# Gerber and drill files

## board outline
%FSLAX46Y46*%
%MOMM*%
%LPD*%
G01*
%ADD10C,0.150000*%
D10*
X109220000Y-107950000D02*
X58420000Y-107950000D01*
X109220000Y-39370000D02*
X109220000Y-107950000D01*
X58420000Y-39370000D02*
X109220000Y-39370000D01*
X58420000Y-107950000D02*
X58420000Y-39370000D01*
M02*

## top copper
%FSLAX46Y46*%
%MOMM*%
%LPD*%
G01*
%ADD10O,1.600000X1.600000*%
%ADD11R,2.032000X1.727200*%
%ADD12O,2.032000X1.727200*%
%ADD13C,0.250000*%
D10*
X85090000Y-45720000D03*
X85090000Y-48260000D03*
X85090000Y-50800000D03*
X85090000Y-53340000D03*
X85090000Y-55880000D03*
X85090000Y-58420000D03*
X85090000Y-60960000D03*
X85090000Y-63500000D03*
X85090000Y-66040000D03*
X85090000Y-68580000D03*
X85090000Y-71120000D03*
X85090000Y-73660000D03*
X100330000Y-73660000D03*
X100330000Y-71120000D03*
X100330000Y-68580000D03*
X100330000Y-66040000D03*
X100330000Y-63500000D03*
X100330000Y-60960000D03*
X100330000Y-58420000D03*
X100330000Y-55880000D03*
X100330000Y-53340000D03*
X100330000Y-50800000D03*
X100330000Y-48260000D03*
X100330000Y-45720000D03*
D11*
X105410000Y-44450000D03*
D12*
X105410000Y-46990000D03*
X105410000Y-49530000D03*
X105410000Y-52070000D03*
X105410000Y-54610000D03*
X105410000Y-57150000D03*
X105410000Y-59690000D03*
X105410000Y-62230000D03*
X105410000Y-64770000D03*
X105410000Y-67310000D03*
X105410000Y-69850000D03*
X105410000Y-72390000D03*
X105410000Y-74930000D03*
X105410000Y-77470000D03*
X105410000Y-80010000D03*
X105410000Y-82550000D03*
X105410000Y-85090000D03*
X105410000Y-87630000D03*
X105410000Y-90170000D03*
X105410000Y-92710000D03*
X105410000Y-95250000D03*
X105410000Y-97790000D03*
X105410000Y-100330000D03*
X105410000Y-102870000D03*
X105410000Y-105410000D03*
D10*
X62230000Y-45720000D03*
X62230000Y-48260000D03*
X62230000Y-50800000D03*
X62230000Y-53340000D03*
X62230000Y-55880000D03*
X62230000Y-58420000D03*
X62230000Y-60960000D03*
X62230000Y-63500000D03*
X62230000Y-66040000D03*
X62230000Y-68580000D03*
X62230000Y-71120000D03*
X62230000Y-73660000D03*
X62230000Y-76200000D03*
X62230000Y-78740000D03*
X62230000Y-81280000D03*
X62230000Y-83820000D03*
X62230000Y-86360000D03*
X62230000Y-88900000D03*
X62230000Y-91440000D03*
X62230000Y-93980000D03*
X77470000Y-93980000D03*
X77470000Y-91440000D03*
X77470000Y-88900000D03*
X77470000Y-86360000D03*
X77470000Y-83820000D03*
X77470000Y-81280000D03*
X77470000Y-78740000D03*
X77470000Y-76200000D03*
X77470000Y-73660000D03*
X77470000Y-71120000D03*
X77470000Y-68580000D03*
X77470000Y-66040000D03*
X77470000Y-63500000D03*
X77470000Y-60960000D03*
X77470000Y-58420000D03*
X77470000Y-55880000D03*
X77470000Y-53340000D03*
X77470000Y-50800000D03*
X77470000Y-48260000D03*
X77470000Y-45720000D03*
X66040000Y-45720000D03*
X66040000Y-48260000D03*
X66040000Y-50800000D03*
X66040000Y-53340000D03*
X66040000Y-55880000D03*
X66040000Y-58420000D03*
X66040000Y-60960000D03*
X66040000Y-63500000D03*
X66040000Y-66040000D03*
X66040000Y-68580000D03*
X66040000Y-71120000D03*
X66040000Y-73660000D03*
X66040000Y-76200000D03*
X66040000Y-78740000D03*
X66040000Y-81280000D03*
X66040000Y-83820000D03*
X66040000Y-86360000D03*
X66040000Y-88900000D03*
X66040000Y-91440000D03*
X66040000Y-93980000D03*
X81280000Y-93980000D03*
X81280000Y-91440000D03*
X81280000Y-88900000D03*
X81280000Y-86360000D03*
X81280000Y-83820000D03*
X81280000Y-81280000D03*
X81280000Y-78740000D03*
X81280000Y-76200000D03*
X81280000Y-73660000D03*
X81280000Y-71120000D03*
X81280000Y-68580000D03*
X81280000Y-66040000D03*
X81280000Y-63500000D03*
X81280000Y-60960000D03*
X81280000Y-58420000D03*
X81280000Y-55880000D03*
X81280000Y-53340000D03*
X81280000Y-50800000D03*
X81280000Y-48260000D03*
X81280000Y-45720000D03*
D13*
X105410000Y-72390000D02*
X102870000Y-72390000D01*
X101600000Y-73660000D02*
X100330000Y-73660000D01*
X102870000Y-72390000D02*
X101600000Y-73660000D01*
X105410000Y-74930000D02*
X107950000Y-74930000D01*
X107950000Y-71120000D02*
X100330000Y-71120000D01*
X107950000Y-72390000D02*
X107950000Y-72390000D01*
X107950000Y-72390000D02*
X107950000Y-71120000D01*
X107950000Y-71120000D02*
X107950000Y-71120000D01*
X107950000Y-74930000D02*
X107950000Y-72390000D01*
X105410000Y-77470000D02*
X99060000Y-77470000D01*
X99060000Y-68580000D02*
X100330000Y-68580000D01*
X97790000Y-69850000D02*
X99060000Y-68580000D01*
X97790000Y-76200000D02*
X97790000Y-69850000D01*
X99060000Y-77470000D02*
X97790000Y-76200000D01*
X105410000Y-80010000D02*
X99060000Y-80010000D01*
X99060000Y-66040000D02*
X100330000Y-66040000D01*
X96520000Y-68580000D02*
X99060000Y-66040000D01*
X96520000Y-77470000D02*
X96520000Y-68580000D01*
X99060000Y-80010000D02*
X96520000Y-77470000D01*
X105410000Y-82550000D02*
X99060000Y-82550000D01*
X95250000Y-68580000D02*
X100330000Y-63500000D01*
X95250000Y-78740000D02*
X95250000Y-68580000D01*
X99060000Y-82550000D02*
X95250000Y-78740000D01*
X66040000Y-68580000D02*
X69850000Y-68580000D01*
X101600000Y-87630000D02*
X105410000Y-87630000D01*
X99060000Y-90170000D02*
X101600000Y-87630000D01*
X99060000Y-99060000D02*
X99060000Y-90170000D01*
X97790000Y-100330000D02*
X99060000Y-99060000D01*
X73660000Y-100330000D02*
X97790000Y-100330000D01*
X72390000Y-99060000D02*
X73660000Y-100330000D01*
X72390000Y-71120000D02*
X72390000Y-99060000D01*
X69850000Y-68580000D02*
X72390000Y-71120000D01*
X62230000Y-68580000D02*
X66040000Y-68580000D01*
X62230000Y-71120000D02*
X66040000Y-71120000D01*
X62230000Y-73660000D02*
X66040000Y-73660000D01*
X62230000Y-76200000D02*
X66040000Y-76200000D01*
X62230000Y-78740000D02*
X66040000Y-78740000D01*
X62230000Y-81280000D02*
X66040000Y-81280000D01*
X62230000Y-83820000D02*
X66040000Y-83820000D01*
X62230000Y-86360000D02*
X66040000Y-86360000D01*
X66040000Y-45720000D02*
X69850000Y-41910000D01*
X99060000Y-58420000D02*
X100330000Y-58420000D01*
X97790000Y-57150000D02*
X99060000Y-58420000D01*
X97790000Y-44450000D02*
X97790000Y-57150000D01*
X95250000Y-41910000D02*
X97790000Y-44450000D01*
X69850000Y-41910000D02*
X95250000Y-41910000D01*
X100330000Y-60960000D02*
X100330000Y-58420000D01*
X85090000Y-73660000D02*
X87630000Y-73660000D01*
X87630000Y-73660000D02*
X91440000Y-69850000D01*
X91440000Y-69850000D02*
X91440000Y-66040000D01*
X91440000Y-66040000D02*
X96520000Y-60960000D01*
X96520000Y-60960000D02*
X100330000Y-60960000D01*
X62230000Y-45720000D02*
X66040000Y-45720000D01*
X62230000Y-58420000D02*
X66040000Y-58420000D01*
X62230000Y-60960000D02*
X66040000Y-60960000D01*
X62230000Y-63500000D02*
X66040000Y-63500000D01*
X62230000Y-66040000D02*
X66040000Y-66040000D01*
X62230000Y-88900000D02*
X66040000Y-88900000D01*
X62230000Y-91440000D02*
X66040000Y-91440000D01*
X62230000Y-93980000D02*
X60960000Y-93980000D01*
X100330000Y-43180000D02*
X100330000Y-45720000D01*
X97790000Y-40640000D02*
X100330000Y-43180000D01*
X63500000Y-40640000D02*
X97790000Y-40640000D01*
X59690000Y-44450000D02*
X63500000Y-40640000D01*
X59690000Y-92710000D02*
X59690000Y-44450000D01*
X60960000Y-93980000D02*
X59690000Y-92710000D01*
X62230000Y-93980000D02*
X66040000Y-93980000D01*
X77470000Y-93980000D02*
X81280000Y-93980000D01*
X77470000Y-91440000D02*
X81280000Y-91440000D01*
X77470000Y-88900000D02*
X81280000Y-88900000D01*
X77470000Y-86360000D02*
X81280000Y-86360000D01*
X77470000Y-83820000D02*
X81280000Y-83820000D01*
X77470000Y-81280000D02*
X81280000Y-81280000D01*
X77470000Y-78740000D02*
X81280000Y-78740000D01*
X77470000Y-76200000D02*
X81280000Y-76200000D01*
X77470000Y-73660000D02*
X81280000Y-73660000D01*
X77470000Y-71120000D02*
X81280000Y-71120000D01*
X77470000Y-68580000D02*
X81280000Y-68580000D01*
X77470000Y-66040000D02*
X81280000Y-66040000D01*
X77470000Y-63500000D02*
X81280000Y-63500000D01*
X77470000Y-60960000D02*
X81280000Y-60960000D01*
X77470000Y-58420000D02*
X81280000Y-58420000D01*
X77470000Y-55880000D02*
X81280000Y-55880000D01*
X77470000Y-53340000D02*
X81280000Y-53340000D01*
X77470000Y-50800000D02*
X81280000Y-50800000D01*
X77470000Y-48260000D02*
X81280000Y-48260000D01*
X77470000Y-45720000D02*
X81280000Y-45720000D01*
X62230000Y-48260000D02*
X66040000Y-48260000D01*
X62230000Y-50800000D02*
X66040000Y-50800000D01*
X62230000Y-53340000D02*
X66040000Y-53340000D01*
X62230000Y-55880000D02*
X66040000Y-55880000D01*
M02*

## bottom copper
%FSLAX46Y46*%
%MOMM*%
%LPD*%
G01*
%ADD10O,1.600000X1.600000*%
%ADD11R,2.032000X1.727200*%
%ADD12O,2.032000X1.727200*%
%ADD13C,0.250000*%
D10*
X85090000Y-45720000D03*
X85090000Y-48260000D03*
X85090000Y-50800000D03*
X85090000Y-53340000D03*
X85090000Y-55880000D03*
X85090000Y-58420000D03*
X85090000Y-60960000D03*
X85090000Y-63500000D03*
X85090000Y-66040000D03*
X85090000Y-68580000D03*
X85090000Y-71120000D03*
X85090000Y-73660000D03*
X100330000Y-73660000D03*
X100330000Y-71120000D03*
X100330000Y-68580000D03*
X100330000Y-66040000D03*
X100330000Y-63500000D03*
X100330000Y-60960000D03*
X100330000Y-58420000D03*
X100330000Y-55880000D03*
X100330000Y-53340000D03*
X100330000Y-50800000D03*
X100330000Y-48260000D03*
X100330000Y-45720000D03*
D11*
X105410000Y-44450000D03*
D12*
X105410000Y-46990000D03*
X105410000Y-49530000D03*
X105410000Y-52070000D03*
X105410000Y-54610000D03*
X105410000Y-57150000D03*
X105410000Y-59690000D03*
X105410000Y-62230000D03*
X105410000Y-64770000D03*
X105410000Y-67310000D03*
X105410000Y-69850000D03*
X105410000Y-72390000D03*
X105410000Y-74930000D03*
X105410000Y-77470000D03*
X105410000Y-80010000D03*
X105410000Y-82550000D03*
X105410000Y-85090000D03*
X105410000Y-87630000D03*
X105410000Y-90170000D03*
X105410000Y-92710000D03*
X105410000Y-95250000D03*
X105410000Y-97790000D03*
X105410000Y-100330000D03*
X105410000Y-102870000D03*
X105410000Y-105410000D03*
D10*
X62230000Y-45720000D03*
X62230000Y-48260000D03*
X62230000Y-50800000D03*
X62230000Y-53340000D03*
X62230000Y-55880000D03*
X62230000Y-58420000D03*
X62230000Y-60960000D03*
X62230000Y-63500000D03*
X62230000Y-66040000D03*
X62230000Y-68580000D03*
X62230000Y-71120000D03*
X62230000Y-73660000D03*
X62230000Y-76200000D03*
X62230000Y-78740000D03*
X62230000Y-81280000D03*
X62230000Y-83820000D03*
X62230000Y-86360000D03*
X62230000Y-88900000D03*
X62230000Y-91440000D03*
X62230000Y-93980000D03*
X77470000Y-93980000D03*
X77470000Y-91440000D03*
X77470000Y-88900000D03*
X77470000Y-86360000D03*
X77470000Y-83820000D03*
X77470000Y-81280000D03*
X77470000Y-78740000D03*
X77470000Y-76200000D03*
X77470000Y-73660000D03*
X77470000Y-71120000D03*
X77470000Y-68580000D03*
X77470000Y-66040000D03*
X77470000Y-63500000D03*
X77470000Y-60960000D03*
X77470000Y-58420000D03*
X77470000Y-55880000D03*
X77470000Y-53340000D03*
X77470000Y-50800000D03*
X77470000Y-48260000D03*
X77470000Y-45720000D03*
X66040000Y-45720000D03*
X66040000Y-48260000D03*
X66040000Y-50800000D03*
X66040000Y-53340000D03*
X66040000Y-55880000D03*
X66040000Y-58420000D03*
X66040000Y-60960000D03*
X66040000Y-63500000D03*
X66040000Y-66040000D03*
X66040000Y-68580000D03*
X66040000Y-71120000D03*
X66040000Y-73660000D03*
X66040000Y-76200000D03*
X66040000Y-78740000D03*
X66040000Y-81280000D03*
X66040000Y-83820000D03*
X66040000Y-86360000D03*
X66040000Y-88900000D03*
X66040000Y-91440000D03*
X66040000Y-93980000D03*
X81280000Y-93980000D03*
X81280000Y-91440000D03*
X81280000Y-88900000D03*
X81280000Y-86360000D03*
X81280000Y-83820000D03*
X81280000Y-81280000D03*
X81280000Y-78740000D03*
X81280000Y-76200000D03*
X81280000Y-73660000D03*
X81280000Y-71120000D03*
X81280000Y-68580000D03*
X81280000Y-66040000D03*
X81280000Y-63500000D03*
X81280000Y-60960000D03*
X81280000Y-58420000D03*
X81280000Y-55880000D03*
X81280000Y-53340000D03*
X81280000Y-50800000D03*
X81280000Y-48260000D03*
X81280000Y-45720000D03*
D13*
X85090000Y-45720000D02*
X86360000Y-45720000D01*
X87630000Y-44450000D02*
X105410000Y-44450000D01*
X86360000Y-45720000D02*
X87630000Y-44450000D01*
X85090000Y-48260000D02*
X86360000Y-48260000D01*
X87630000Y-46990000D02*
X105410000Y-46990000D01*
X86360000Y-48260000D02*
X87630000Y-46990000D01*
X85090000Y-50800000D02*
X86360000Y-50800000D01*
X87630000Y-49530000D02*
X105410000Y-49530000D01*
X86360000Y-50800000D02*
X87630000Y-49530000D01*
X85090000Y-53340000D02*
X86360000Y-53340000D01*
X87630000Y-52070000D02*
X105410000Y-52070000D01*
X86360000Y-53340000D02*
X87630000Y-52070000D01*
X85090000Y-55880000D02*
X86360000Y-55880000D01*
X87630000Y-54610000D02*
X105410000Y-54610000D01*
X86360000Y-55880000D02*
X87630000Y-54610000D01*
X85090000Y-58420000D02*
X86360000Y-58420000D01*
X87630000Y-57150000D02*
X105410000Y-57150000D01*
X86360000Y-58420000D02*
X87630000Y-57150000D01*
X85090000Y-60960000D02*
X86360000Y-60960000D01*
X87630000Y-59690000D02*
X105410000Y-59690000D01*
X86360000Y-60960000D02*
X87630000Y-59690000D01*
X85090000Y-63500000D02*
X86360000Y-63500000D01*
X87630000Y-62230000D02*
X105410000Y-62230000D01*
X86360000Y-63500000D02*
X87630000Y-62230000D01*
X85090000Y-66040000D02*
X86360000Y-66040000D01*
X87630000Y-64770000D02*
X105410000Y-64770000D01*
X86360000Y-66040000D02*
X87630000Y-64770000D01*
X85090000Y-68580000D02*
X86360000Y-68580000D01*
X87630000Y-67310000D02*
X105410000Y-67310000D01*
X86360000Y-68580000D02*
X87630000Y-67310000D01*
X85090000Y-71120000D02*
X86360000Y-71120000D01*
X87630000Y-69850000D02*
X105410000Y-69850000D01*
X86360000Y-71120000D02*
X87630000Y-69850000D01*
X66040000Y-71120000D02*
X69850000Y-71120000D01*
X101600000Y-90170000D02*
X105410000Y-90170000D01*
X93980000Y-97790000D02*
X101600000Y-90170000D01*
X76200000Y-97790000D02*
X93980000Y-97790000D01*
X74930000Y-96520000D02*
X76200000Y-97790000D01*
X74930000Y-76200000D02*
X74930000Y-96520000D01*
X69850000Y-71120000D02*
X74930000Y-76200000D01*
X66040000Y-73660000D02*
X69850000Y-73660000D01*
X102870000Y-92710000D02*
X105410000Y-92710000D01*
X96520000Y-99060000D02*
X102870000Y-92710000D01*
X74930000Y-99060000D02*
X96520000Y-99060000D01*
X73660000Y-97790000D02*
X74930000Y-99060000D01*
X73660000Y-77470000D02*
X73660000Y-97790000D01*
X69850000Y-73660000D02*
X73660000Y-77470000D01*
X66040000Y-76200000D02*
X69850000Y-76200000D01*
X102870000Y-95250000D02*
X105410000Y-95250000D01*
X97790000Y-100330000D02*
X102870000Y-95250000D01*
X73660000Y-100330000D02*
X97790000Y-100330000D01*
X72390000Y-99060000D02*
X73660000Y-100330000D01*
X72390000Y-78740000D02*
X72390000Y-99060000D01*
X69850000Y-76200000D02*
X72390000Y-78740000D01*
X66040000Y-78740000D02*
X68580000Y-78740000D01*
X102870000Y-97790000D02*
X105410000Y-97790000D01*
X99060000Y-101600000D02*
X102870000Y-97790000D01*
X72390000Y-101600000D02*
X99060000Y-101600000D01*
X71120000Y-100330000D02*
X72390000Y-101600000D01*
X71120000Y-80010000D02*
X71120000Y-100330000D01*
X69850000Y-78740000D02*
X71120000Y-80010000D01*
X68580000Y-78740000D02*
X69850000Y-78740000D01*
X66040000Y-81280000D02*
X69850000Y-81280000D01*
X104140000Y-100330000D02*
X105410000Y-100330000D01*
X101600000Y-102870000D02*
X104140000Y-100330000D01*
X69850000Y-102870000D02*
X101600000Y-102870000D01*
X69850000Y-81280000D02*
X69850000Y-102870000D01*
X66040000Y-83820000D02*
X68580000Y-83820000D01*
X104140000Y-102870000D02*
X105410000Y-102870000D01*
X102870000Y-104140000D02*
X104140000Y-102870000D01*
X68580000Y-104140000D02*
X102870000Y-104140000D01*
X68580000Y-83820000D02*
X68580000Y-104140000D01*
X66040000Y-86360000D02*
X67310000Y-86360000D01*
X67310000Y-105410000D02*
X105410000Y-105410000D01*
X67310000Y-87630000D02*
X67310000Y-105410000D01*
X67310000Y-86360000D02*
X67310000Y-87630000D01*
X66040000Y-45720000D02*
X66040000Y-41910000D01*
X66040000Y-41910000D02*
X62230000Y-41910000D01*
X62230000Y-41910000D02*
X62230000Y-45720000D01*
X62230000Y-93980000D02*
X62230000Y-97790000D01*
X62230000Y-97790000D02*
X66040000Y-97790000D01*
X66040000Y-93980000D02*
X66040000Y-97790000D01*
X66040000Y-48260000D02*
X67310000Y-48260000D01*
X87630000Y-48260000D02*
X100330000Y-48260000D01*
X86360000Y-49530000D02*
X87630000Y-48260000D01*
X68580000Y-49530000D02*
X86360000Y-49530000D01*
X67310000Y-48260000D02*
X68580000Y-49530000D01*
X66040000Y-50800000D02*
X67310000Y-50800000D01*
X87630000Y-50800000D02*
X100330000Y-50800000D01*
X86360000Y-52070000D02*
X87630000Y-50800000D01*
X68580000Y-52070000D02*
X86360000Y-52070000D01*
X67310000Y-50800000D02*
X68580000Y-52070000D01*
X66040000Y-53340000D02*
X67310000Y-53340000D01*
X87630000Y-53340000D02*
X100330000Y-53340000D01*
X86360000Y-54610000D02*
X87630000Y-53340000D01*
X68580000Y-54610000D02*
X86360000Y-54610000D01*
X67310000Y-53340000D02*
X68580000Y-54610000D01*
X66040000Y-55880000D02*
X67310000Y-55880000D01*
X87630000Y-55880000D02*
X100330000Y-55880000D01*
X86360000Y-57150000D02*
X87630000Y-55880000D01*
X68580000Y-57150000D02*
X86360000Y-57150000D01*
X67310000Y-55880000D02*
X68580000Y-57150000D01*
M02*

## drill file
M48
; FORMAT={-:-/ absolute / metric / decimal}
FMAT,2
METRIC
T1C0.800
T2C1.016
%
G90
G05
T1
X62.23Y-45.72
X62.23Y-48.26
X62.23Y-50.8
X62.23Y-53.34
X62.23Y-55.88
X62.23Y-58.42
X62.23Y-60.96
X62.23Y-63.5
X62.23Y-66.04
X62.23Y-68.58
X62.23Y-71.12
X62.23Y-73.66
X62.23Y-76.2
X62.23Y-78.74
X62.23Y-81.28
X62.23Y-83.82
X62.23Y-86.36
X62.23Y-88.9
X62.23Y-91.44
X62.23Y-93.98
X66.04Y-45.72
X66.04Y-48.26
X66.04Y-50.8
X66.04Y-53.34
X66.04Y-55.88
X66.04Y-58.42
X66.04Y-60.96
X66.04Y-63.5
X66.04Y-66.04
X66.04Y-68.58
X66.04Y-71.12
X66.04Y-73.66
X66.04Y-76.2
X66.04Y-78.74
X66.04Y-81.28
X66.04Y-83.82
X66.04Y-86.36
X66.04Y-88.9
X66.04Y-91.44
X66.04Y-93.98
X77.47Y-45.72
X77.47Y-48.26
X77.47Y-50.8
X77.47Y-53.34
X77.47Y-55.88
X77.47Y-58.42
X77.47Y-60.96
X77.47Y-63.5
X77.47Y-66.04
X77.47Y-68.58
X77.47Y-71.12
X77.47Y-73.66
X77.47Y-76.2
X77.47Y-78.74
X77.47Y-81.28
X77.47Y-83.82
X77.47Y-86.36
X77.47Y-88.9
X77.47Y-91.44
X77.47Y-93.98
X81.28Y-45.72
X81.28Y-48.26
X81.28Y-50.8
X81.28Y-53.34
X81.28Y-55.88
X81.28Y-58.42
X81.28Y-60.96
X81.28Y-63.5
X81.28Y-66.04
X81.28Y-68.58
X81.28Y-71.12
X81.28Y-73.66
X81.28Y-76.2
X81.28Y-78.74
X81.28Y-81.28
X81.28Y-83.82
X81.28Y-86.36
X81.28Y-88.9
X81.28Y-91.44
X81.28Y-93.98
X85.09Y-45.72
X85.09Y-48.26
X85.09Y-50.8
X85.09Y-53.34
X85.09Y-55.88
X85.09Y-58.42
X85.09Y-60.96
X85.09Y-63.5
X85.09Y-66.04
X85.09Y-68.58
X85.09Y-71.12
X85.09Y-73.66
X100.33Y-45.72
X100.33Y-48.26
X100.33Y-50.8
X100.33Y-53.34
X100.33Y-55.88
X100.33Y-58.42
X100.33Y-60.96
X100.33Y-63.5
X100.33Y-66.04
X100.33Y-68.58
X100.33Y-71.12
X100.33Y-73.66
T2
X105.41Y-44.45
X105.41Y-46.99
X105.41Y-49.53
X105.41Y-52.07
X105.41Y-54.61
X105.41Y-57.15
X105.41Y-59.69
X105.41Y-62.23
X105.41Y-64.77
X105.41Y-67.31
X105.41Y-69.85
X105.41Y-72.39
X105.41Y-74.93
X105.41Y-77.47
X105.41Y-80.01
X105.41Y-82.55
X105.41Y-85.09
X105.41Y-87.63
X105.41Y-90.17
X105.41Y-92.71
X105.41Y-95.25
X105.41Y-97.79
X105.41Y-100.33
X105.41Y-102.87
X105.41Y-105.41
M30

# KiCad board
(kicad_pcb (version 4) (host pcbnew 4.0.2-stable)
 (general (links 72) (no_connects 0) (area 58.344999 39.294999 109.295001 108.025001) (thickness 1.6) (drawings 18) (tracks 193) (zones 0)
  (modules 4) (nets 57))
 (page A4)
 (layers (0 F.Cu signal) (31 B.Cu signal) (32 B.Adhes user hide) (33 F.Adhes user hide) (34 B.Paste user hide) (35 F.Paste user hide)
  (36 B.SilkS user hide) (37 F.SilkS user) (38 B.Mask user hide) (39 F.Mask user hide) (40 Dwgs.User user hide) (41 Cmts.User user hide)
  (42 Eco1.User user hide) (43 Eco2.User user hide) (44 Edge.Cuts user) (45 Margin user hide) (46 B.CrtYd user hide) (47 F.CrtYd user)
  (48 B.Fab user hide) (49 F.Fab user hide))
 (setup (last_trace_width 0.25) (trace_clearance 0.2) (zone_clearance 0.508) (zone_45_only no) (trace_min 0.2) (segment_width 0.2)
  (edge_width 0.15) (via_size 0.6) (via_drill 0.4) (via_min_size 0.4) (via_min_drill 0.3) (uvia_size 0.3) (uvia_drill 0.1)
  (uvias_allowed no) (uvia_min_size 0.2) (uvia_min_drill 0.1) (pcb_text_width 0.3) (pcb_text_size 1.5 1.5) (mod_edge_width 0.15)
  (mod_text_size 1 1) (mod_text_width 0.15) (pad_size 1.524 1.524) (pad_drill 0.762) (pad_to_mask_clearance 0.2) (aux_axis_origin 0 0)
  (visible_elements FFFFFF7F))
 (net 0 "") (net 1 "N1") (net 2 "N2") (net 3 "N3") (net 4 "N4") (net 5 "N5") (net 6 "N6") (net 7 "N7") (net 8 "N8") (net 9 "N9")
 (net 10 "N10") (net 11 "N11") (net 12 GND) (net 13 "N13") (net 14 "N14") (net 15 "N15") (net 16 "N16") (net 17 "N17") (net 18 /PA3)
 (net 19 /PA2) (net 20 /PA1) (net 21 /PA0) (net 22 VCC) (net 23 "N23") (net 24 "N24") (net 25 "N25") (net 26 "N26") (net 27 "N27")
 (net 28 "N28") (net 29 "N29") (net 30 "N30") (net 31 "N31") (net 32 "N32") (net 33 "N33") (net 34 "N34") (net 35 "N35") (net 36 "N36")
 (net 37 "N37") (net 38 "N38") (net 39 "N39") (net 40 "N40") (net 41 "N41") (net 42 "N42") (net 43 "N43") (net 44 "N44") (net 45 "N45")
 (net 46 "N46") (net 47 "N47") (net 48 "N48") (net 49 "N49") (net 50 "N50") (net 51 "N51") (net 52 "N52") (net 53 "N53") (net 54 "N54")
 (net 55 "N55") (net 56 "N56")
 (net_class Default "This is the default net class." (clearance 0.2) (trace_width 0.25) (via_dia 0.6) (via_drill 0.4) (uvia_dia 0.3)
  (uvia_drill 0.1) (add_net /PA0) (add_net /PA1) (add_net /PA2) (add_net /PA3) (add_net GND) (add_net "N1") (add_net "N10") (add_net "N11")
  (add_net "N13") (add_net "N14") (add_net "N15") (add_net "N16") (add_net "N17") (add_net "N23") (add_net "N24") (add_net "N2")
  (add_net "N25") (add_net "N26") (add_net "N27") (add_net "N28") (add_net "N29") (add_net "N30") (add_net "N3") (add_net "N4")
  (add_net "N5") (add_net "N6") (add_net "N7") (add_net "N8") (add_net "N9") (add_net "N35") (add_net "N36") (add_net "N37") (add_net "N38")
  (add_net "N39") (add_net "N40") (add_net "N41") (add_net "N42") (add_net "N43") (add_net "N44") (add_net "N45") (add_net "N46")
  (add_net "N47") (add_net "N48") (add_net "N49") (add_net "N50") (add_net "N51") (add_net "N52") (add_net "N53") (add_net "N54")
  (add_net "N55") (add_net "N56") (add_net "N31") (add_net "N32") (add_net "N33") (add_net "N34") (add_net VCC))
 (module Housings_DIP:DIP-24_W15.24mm (layer F.Cu) (at 85.09 45.72)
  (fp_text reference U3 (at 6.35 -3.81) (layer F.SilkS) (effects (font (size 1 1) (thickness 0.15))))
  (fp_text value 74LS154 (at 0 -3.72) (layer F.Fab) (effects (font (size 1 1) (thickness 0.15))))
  (pad 1 thru_hole oval (at 0 0) (size 1.6 1.6) (drill 0.8) (layers *.Cu *.Mask F.SilkS) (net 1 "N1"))
  (pad 2 thru_hole oval (at 0 2.54) (size 1.6 1.6) (drill 0.8) (layers *.Cu *.Mask F.SilkS) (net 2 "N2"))
  (pad 3 thru_hole oval (at 0 5.08) (size 1.6 1.6) (drill 0.8) (layers *.Cu *.Mask F.SilkS) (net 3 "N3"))
  (pad 4 thru_hole oval (at 0 7.62) (size 1.6 1.6) (drill 0.8) (layers *.Cu *.Mask F.SilkS) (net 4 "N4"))
  (pad 5 thru_hole oval (at 0 10.16) (size 1.6 1.6) (drill 0.8) (layers *.Cu *.Mask F.SilkS) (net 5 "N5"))
  (pad 6 thru_hole oval (at 0 12.7) (size 1.6 1.6) (drill 0.8) (layers *.Cu *.Mask F.SilkS) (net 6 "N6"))
  (pad 7 thru_hole oval (at 0 15.24) (size 1.6 1.6) (drill 0.8) (layers *.Cu *.Mask F.SilkS) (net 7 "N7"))
  (pad 8 thru_hole oval (at 0 17.78) (size 1.6 1.6) (drill 0.8) (layers *.Cu *.Mask F.SilkS) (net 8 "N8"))
  (pad 9 thru_hole oval (at 0 20.32) (size 1.6 1.6) (drill 0.8) (layers *.Cu *.Mask F.SilkS) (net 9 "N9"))
  (pad 10 thru_hole oval (at 0 22.86) (size 1.6 1.6) (drill 0.8) (layers *.Cu *.Mask F.SilkS) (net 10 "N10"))
  (pad 11 thru_hole oval (at 0 25.4) (size 1.6 1.6) (drill 0.8) (layers *.Cu *.Mask F.SilkS) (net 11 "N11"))
  (pad 12 thru_hole oval (at 0 27.94) (size 1.6 1.6) (drill 0.8) (layers *.Cu *.Mask F.SilkS) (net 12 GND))
  (pad 13 thru_hole oval (at 15.24 27.94) (size 1.6 1.6) (drill 0.8) (layers *.Cu *.Mask F.SilkS) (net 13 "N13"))
  (pad 14 thru_hole oval (at 15.24 25.4) (size 1.6 1.6) (drill 0.8) (layers *.Cu *.Mask F.SilkS) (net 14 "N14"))
  (pad 15 thru_hole oval (at 15.24 22.86) (size 1.6 1.6) (drill 0.8) (layers *.Cu *.Mask F.SilkS) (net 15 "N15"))
  (pad 16 thru_hole oval (at 15.24 20.32) (size 1.6 1.6) (drill 0.8) (layers *.Cu *.Mask F.SilkS) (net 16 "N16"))
  (pad 17 thru_hole oval (at 15.24 17.78) (size 1.6 1.6) (drill 0.8) (layers *.Cu *.Mask F.SilkS) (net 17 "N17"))
  (pad 18 thru_hole oval (at 15.24 15.24) (size 1.6 1.6) (drill 0.8) (layers *.Cu *.Mask F.SilkS) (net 12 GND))
  (pad 19 thru_hole oval (at 15.24 12.7) (size 1.6 1.6) (drill 0.8) (layers *.Cu *.Mask F.SilkS) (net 12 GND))
  (pad 20 thru_hole oval (at 15.24 10.16) (size 1.6 1.6) (drill 0.8) (layers *.Cu *.Mask F.SilkS) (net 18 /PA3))
  (pad 21 thru_hole oval (at 15.24 7.62) (size 1.6 1.6) (drill 0.8) (layers *.Cu *.Mask F.SilkS) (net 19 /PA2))
  (pad 22 thru_hole oval (at 15.24 5.08) (size 1.6 1.6) (drill 0.8) (layers *.Cu *.Mask F.SilkS) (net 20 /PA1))
  (pad 23 thru_hole oval (at 15.24 2.54) (size 1.6 1.6) (drill 0.8) (layers *.Cu *.Mask F.SilkS) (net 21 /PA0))
  (pad 24 thru_hole oval (at 15.24 0) (size 1.6 1.6) (drill 0.8) (layers *.Cu *.Mask F.SilkS) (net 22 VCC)))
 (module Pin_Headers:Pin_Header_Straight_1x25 (layer F.Cu) (at 105.41 44.45)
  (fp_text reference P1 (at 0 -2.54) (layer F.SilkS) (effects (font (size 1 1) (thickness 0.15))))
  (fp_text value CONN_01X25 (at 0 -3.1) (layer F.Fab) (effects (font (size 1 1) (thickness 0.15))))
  (pad 1 thru_hole rect (at 0 0) (size 2.032 1.7272) (drill 1.016) (layers *.Cu *.Mask F.SilkS) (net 1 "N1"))
  (pad 2 thru_hole oval (at 0 2.54) (size 2.032 1.7272) (drill 1.016) (layers *.Cu *.Mask F.SilkS) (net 2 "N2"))
  (pad 3 thru_hole oval (at 0 5.08) (size 2.032 1.7272) (drill 1.016) (layers *.Cu *.Mask F.SilkS) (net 3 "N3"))
  (pad 4 thru_hole oval (at 0 7.62) (size 2.032 1.7272) (drill 1.016) (layers *.Cu *.Mask F.SilkS) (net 4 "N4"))
  (pad 5 thru_hole oval (at 0 10.16) (size 2.032 1.7272) (drill 1.016) (layers *.Cu *.Mask F.SilkS) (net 5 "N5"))
  (pad 6 thru_hole oval (at 0 12.7) (size 2.032 1.7272) (drill 1.016) (layers *.Cu *.Mask F.SilkS) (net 6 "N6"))
  (pad 7 thru_hole oval (at 0 15.24) (size 2.032 1.7272) (drill 1.016) (layers *.Cu *.Mask F.SilkS) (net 7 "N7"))
  (pad 8 thru_hole oval (at 0 17.78) (size 2.032 1.7272) (drill 1.016) (layers *.Cu *.Mask F.SilkS) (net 8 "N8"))
  (pad 9 thru_hole oval (at 0 20.32) (size 2.032 1.7272) (drill 1.016) (layers *.Cu *.Mask F.SilkS) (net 9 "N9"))
  (pad 10 thru_hole oval (at 0 22.86) (size 2.032 1.7272) (drill 1.016) (layers *.Cu *.Mask F.SilkS) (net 10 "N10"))
  (pad 11 thru_hole oval (at 0 25.4) (size 2.032 1.7272) (drill 1.016) (layers *.Cu *.Mask F.SilkS) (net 11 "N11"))
  (pad 12 thru_hole oval (at 0 27.94) (size 2.032 1.7272) (drill 1.016) (layers *.Cu *.Mask F.SilkS) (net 13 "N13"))
  (pad 13 thru_hole oval (at 0 30.48) (size 2.032 1.7272) (drill 1.016) (layers *.Cu *.Mask F.SilkS) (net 14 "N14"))
  (pad 14 thru_hole oval (at 0 33.02) (size 2.032 1.7272) (drill 1.016) (layers *.Cu *.Mask F.SilkS) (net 15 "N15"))
  (pad 15 thru_hole oval (at 0 35.56) (size 2.032 1.7272) (drill 1.016) (layers *.Cu *.Mask F.SilkS) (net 16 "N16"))
  (pad 16 thru_hole oval (at 0 38.1) (size 2.032 1.7272) (drill 1.016) (layers *.Cu *.Mask F.SilkS) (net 17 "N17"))
  (pad 17 thru_hole oval (at 0 40.64) (size 2.032 1.7272) (drill 1.016) (layers *.Cu *.Mask F.SilkS))
  (pad 18 thru_hole oval (at 0 43.18) (size 2.032 1.7272) (drill 1.016) (layers *.Cu *.Mask F.SilkS) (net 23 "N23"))
  (pad 19 thru_hole oval (at 0 45.72) (size 2.032 1.7272) (drill 1.016) (layers *.Cu *.Mask F.SilkS) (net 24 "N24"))
  (pad 20 thru_hole oval (at 0 48.26) (size 2.032 1.7272) (drill 1.016) (layers *.Cu *.Mask F.SilkS) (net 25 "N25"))
  (pad 21 thru_hole oval (at 0 50.8) (size 2.032 1.7272) (drill 1.016) (layers *.Cu *.Mask F.SilkS) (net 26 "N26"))
  (pad 22 thru_hole oval (at 0 53.34) (size 2.032 1.7272) (drill 1.016) (layers *.Cu *.Mask F.SilkS) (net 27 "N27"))
  (pad 23 thru_hole oval (at 0 55.88) (size 2.032 1.7272) (drill 1.016) (layers *.Cu *.Mask F.SilkS) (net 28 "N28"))
  (pad 24 thru_hole oval (at 0 58.42) (size 2.032 1.7272) (drill 1.016) (layers *.Cu *.Mask F.SilkS) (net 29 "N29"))
  (pad 25 thru_hole oval (at 0 60.96) (size 2.032 1.7272) (drill 1.016) (layers *.Cu *.Mask F.SilkS) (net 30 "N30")))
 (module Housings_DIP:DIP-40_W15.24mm (layer F.Cu) (at 62.23 45.72)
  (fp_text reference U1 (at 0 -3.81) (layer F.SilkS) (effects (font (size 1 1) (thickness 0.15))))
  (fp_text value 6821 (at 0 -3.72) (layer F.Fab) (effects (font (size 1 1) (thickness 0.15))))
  (pad 1 thru_hole oval (at 0 0) (size 1.6 1.6) (drill 0.8) (layers *.Cu *.Mask F.SilkS) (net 12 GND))
  (pad 2 thru_hole oval (at 0 2.54) (size 1.6 1.6) (drill 0.8) (layers *.Cu *.Mask F.SilkS) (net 21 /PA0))
  (pad 3 thru_hole oval (at 0 5.08) (size 1.6 1.6) (drill 0.8) (layers *.Cu *.Mask F.SilkS) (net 20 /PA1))
  (pad 4 thru_hole oval (at 0 7.62) (size 1.6 1.6) (drill 0.8) (layers *.Cu *.Mask F.SilkS) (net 19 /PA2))
  (pad 5 thru_hole oval (at 0 10.16) (size 1.6 1.6) (drill 0.8) (layers *.Cu *.Mask F.SilkS) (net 18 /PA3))
  (pad 6 thru_hole oval (at 0 12.7) (size 1.6 1.6) (drill 0.8) (layers *.Cu *.Mask F.SilkS) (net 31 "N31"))
  (pad 7 thru_hole oval (at 0 15.24) (size 1.6 1.6) (drill 0.8) (layers *.Cu *.Mask F.SilkS) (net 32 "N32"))
  (pad 8 thru_hole oval (at 0 17.78) (size 1.6 1.6) (drill 0.8) (layers *.Cu *.Mask F.SilkS) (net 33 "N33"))
  (pad 9 thru_hole oval (at 0 20.32) (size 1.6 1.6) (drill 0.8) (layers *.Cu *.Mask F.SilkS) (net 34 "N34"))
  (pad 10 thru_hole oval (at 0 22.86) (size 1.6 1.6) (drill 0.8) (layers *.Cu *.Mask F.SilkS) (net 23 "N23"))
  (pad 11 thru_hole oval (at 0 25.4) (size 1.6 1.6) (drill 0.8) (layers *.Cu *.Mask F.SilkS) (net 24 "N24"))
  (pad 12 thru_hole oval (at 0 27.94) (size 1.6 1.6) (drill 0.8) (layers *.Cu *.Mask F.SilkS) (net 25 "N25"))
  (pad 13 thru_hole oval (at 0 30.48) (size 1.6 1.6) (drill 0.8) (layers *.Cu *.Mask F.SilkS) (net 26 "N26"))
  (pad 14 thru_hole oval (at 0 33.02) (size 1.6 1.6) (drill 0.8) (layers *.Cu *.Mask F.SilkS) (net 27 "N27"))
  (pad 15 thru_hole oval (at 0 35.56) (size 1.6 1.6) (drill 0.8) (layers *.Cu *.Mask F.SilkS) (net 28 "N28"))
  (pad 16 thru_hole oval (at 0 38.1) (size 1.6 1.6) (drill 0.8) (layers *.Cu *.Mask F.SilkS) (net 29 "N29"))
  (pad 17 thru_hole oval (at 0 40.64) (size 1.6 1.6) (drill 0.8) (layers *.Cu *.Mask F.SilkS) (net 30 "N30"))
  (pad 18 thru_hole oval (at 0 43.18) (size 1.6 1.6) (drill 0.8) (layers *.Cu *.Mask F.SilkS) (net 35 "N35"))
  (pad 19 thru_hole oval (at 0 45.72) (size 1.6 1.6) (drill 0.8) (layers *.Cu *.Mask F.SilkS) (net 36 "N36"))
  (pad 20 thru_hole oval (at 0 48.26) (size 1.6 1.6) (drill 0.8) (layers *.Cu *.Mask F.SilkS) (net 22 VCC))
  (pad 21 thru_hole oval (at 15.24 48.26) (size 1.6 1.6) (drill 0.8) (layers *.Cu *.Mask F.SilkS) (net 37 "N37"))
  (pad 22 thru_hole oval (at 15.24 45.72) (size 1.6 1.6) (drill 0.8) (layers *.Cu *.Mask F.SilkS) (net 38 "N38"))
  (pad 23 thru_hole oval (at 15.24 43.18) (size 1.6 1.6) (drill 0.8) (layers *.Cu *.Mask F.SilkS) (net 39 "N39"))
  (pad 24 thru_hole oval (at 15.24 40.64) (size 1.6 1.6) (drill 0.8) (layers *.Cu *.Mask F.SilkS) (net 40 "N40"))
  (pad 25 thru_hole oval (at 15.24 38.1) (size 1.6 1.6) (drill 0.8) (layers *.Cu *.Mask F.SilkS) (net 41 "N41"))
  (pad 26 thru_hole oval (at 15.24 35.56) (size 1.6 1.6) (drill 0.8) (layers *.Cu *.Mask F.SilkS) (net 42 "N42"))
  (pad 27 thru_hole oval (at 15.24 33.02) (size 1.6 1.6) (drill 0.8) (layers *.Cu *.Mask F.SilkS) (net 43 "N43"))
  (pad 28 thru_hole oval (at 15.24 30.48) (size 1.6 1.6) (drill 0.8) (layers *.Cu *.Mask F.SilkS) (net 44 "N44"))
  (pad 29 thru_hole oval (at 15.24 27.94) (size 1.6 1.6) (drill 0.8) (layers *.Cu *.Mask F.SilkS) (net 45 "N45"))
  (pad 30 thru_hole oval (at 15.24 25.4) (size 1.6 1.6) (drill 0.8) (layers *.Cu *.Mask F.SilkS) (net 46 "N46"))
  (pad 31 thru_hole oval (at 15.24 22.86) (size 1.6 1.6) (drill 0.8) (layers *.Cu *.Mask F.SilkS) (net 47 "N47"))
  (pad 32 thru_hole oval (at 15.24 20.32) (size 1.6 1.6) (drill 0.8) (layers *.Cu *.Mask F.SilkS) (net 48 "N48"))
  (pad 33 thru_hole oval (at 15.24 17.78) (size 1.6 1.6) (drill 0.8) (layers *.Cu *.Mask F.SilkS) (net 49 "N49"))
  (pad 34 thru_hole oval (at 15.24 15.24) (size 1.6 1.6) (drill 0.8) (layers *.Cu *.Mask F.SilkS) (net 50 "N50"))
  (pad 35 thru_hole oval (at 15.24 12.7) (size 1.6 1.6) (drill 0.8) (layers *.Cu *.Mask F.SilkS) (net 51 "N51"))
  (pad 36 thru_hole oval (at 15.24 10.16) (size 1.6 1.6) (drill 0.8) (layers *.Cu *.Mask F.SilkS) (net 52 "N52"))
  (pad 37 thru_hole oval (at 15.24 7.62) (size 1.6 1.6) (drill 0.8) (layers *.Cu *.Mask F.SilkS) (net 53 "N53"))
  (pad 38 thru_hole oval (at 15.24 5.08) (size 1.6 1.6) (drill 0.8) (layers *.Cu *.Mask F.SilkS) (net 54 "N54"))
  (pad 39 thru_hole oval (at 15.24 2.54) (size 1.6 1.6) (drill 0.8) (layers *.Cu *.Mask F.SilkS) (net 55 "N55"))
  (pad 40 thru_hole oval (at 15.24 0) (size 1.6 1.6) (drill 0.8) (layers *.Cu *.Mask F.SilkS) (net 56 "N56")))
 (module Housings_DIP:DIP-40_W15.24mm (layer F.Cu) (at 66.04 45.72)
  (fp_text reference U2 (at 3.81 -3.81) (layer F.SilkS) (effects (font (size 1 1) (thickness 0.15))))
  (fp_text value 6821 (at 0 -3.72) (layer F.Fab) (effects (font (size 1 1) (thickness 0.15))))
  (pad 1 thru_hole oval (at 0 0) (size 1.6 1.6) (drill 0.8) (layers *.Cu *.Mask F.SilkS) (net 12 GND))
  (pad 2 thru_hole oval (at 0 2.54) (size 1.6 1.6) (drill 0.8) (layers *.Cu *.Mask F.SilkS) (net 21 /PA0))
  (pad 3 thru_hole oval (at 0 5.08) (size 1.6 1.6) (drill 0.8) (layers *.Cu *.Mask F.SilkS) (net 20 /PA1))
  (pad 4 thru_hole oval (at 0 7.62) (size 1.6 1.6) (drill 0.8) (layers *.Cu *.Mask F.SilkS) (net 19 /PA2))
  (pad 5 thru_hole oval (at 0 10.16) (size 1.6 1.6) (drill 0.8) (layers *.Cu *.Mask F.SilkS) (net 18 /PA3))
  (pad 6 thru_hole oval (at 0 12.7) (size 1.6 1.6) (drill 0.8) (layers *.Cu *.Mask F.SilkS) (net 31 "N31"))
  (pad 7 thru_hole oval (at 0 15.24) (size 1.6 1.6) (drill 0.8) (layers *.Cu *.Mask F.SilkS) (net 32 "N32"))
  (pad 8 thru_hole oval (at 0 17.78) (size 1.6 1.6) (drill 0.8) (layers *.Cu *.Mask F.SilkS) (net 33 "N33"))
  (pad 9 thru_hole oval (at 0 20.32) (size 1.6 1.6) (drill 0.8) (layers *.Cu *.Mask F.SilkS) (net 34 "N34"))
  (pad 10 thru_hole oval (at 0 22.86) (size 1.6 1.6) (drill 0.8) (layers *.Cu *.Mask F.SilkS) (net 23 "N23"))
  (pad 11 thru_hole oval (at 0 25.4) (size 1.6 1.6) (drill 0.8) (layers *.Cu *.Mask F.SilkS) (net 24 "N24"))
  (pad 12 thru_hole oval (at 0 27.94) (size 1.6 1.6) (drill 0.8) (layers *.Cu *.Mask F.SilkS) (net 25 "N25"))
  (pad 13 thru_hole oval (at 0 30.48) (size 1.6 1.6) (drill 0.8) (layers *.Cu *.Mask F.SilkS) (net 26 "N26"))
  (pad 14 thru_hole oval (at 0 33.02) (size 1.6 1.6) (drill 0.8) (layers *.Cu *.Mask F.SilkS) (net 27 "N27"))
  (pad 15 thru_hole oval (at 0 35.56) (size 1.6 1.6) (drill 0.8) (layers *.Cu *.Mask F.SilkS) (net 28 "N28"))
  (pad 16 thru_hole oval (at 0 38.1) (size 1.6 1.6) (drill 0.8) (layers *.Cu *.Mask F.SilkS) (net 29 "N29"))
  (pad 17 thru_hole oval (at 0 40.64) (size 1.6 1.6) (drill 0.8) (layers *.Cu *.Mask F.SilkS) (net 30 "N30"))
  (pad 18 thru_hole oval (at 0 43.18) (size 1.6 1.6) (drill 0.8) (layers *.Cu *.Mask F.SilkS) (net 35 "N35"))
  (pad 19 thru_hole oval (at 0 45.72) (size 1.6 1.6) (drill 0.8) (layers *.Cu *.Mask F.SilkS) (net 36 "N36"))
  (pad 20 thru_hole oval (at 0 48.26) (size 1.6 1.6) (drill 0.8) (layers *.Cu *.Mask F.SilkS) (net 22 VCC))
  (pad 21 thru_hole oval (at 15.24 48.26) (size 1.6 1.6) (drill 0.8) (layers *.Cu *.Mask F.SilkS) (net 37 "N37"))
  (pad 22 thru_hole oval (at 15.24 45.72) (size 1.6 1.6) (drill 0.8) (layers *.Cu *.Mask F.SilkS) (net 38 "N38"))
  (pad 23 thru_hole oval (at 15.24 43.18) (size 1.6 1.6) (drill 0.8) (layers *.Cu *.Mask F.SilkS) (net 39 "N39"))
  (pad 24 thru_hole oval (at 15.24 40.64) (size 1.6 1.6) (drill 0.8) (layers *.Cu *.Mask F.SilkS) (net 40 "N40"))
  (pad 25 thru_hole oval (at 15.24 38.1) (size 1.6 1.6) (drill 0.8) (layers *.Cu *.Mask F.SilkS) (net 41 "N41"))
  (pad 26 thru_hole oval (at 15.24 35.56) (size 1.6 1.6) (drill 0.8) (layers *.Cu *.Mask F.SilkS) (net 42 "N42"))
  (pad 27 thru_hole oval (at 15.24 33.02) (size 1.6 1.6) (drill 0.8) (layers *.Cu *.Mask F.SilkS) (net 43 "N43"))
  (pad 28 thru_hole oval (at 15.24 30.48) (size 1.6 1.6) (drill 0.8) (layers *.Cu *.Mask F.SilkS) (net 44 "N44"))
  (pad 29 thru_hole oval (at 15.24 27.94) (size 1.6 1.6) (drill 0.8) (layers *.Cu *.Mask F.SilkS) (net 45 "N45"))
  (pad 30 thru_hole oval (at 15.24 25.4) (size 1.6 1.6) (drill 0.8) (layers *.Cu *.Mask F.SilkS) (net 46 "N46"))
  (pad 31 thru_hole oval (at 15.24 22.86) (size 1.6 1.6) (drill 0.8) (layers *.Cu *.Mask F.SilkS) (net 47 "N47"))
  (pad 32 thru_hole oval (at 15.24 20.32) (size 1.6 1.6) (drill 0.8) (layers *.Cu *.Mask F.SilkS) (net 48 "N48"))
  (pad 33 thru_hole oval (at 15.24 17.78) (size 1.6 1.6) (drill 0.8) (layers *.Cu *.Mask F.SilkS) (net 49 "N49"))
  (pad 34 thru_hole oval (at 15.24 15.24) (size 1.6 1.6) (drill 0.8) (layers *.Cu *.Mask F.SilkS) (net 50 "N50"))
  (pad 35 thru_hole oval (at 15.24 12.7) (size 1.6 1.6) (drill 0.8) (layers *.Cu *.Mask F.SilkS) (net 51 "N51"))
  (pad 36 thru_hole oval (at 15.24 10.16) (size 1.6 1.6) (drill 0.8) (layers *.Cu *.Mask F.SilkS) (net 52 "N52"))
  (pad 37 thru_hole oval (at 15.24 7.62) (size 1.6 1.6) (drill 0.8) (layers *.Cu *.Mask F.SilkS) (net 53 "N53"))
  (pad 38 thru_hole oval (at 15.24 5.08) (size 1.6 1.6) (drill 0.8) (layers *.Cu *.Mask F.SilkS) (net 54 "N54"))
  (pad 39 thru_hole oval (at 15.24 2.54) (size 1.6 1.6) (drill 0.8) (layers *.Cu *.Mask F.SilkS) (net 55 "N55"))
  (pad 40 thru_hole oval (at 15.24 0) (size 1.6 1.6) (drill 0.8) (layers *.Cu *.Mask F.SilkS) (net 56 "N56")))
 (gr_line (start 109.22 107.95) (end 58.42 107.95) (angle 90) (layer Edge.Cuts) (width 0.15))
 (gr_line (start 109.22 39.37) (end 109.22 107.95) (angle 90) (layer Edge.Cuts) (width 0.15))
 (gr_line (start 58.42 39.37) (end 109.22 39.37) (angle 90) (layer Edge.Cuts) (width 0.15))
 (gr_line (start 58.42 107.95) (end 58.42 39.37) (angle 90) (layer Edge.Cuts) (width 0.15))
 (segment (start 85.09 45.72) (end 86.36 45.72) (width 0.25) (layer B.Cu) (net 1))
 (segment (start 87.63 44.45) (end 105.41 44.45) (width 0.25) (layer B.Cu) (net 1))
 (segment (start 86.36 45.72) (end 87.63 44.45) (width 0.25) (layer B.Cu) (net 1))
 (segment (start 85.09 48.26) (end 86.36 48.26) (width 0.25) (layer B.Cu) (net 2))
 (segment (start 87.63 46.99) (end 105.41 46.99) (width 0.25) (layer B.Cu) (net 2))
 (segment (start 86.36 48.26) (end 87.63 46.99) (width 0.25) (layer B.Cu) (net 2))
 (segment (start 85.09 50.8) (end 86.36 50.8) (width 0.25) (layer B.Cu) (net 3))
 (segment (start 87.63 49.53) (end 105.41 49.53) (width 0.25) (layer B.Cu) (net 3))
 (segment (start 86.36 50.8) (end 87.63 49.53) (width 0.25) (layer B.Cu) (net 3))
 (segment (start 85.09 53.34) (end 86.36 53.34) (width 0.25) (layer B.Cu) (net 4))
 (segment (start 87.63 52.07) (end 105.41 52.07) (width 0.25) (layer B.Cu) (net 4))
 (segment (start 86.36 53.34) (end 87.63 52.07) (width 0.25) (layer B.Cu) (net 4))
 (segment (start 85.09 55.88) (end 86.36 55.88) (width 0.25) (layer B.Cu) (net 5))
 (segment (start 87.63 54.61) (end 105.41 54.61) (width 0.25) (layer B.Cu) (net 5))
 (segment (start 86.36 55.88) (end 87.63 54.61) (width 0.25) (layer B.Cu) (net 5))
 (segment (start 85.09 58.42) (end 86.36 58.42) (width 0.25) (layer B.Cu) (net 6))
 (segment (start 87.63 57.15) (end 105.41 57.15) (width 0.25) (layer B.Cu) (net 6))
 (segment (start 86.36 58.42) (end 87.63 57.15) (width 0.25) (layer B.Cu) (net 6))
 (segment (start 85.09 60.96) (end 86.36 60.96) (width 0.25) (layer B.Cu) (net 7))
 (segment (start 87.63 59.69) (end 105.41 59.69) (width 0.25) (layer B.Cu) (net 7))
 (segment (start 86.36 60.96) (end 87.63 59.69) (width 0.25) (layer B.Cu) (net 7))
 (segment (start 85.09 63.5) (end 86.36 63.5) (width 0.25) (layer B.Cu) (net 8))
 (segment (start 87.63 62.23) (end 105.41 62.23) (width 0.25) (layer B.Cu) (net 8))
 (segment (start 86.36 63.5) (end 87.63 62.23) (width 0.25) (layer B.Cu) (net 8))
 (segment (start 85.09 66.04) (end 86.36 66.04) (width 0.25) (layer B.Cu) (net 9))
 (segment (start 87.63 64.77) (end 105.41 64.77) (width 0.25) (layer B.Cu) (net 9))
 (segment (start 86.36 66.04) (end 87.63 64.77) (width 0.25) (layer B.Cu) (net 9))
 (segment (start 85.09 68.58) (end 86.36 68.58) (width 0.25) (layer B.Cu) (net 10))
 (segment (start 87.63 67.31) (end 105.41 67.31) (width 0.25) (layer B.Cu) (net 10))
 (segment (start 86.36 68.58) (end 87.63 67.31) (width 0.25) (layer B.Cu) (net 10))
 (segment (start 85.09 71.12) (end 86.36 71.12) (width 0.25) (layer B.Cu) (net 11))
 (segment (start 87.63 69.85) (end 105.41 69.85) (width 0.25) (layer B.Cu) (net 11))
 (segment (start 86.36 71.12) (end 87.63 69.85) (width 0.25) (layer B.Cu) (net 11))
 (segment (start 105.41 72.39) (end 102.87 72.39) (width 0.25) (layer F.Cu) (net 13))
 (segment (start 101.6 73.66) (end 100.33 73.66) (width 0.25) (layer F.Cu) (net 13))
 (segment (start 102.87 72.39) (end 101.6 73.66) (width 0.25) (layer F.Cu) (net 13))
 (segment (start 105.41 74.93) (end 107.95 74.93) (width 0.25) (layer F.Cu) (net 14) (status 400000))
 (segment (start 107.95 71.12) (end 100.33 71.12) (width 0.25) (layer F.Cu) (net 14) (status 800000))
 (segment (start 107.95 72.39) (end 107.95 72.39) (width 0.25) (layer F.Cu) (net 14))
 (segment (start 107.95 72.39) (end 107.95 71.12) (width 0.25) (layer F.Cu) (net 14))
 (segment (start 107.95 71.12) (end 107.95 71.12) (width 0.25) (layer F.Cu) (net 14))
 (segment (start 107.95 74.93) (end 107.95 72.39) (width 0.25) (layer F.Cu) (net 14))
 (segment (start 105.41 77.47) (end 99.06 77.47) (width 0.25) (layer F.Cu) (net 15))
 (segment (start 99.06 68.58) (end 100.33 68.58) (width 0.25) (layer F.Cu) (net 15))
 (segment (start 97.79 69.85) (end 99.06 68.58) (width 0.25) (layer F.Cu) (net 15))
 (segment (start 97.79 76.2) (end 97.79 69.85) (width 0.25) (layer F.Cu) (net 15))
 (segment (start 99.06 77.47) (end 97.79 76.2) (width 0.25) (layer F.Cu) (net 15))
 (segment (start 105.41 80.01) (end 99.06 80.01) (width 0.25) (layer F.Cu) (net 16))
 (segment (start 99.06 66.04) (end 100.33 66.04) (width 0.25) (layer F.Cu) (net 16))
 (segment (start 96.52 68.58) (end 99.06 66.04) (width 0.25) (layer F.Cu) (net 16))
 (segment (start 96.52 77.47) (end 96.52 68.58) (width 0.25) (layer F.Cu) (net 16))
 (segment (start 99.06 80.01) (end 96.52 77.47) (width 0.25) (layer F.Cu) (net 16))
 (segment (start 105.41 82.55) (end 99.06 82.55) (width 0.25) (layer F.Cu) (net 17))
 (segment (start 95.25 68.58) (end 100.33 63.5) (width 0.25) (layer F.Cu) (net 17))
 (segment (start 95.25 78.74) (end 95.25 68.58) (width 0.25) (layer F.Cu) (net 17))
 (segment (start 99.06 82.55) (end 95.25 78.74) (width 0.25) (layer F.Cu) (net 17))
 (segment (start 66.04 68.58) (end 69.85 68.58) (width 0.25) (layer F.Cu) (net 23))
 (segment (start 101.6 87.63) (end 105.41 87.63) (width 0.25) (layer F.Cu) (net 23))
 (segment (start 99.06 90.17) (end 101.6 87.63) (width 0.25) (layer F.Cu) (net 23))
 (segment (start 99.06 99.06) (end 99.06 90.17) (width 0.25) (layer F.Cu) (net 23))
 (segment (start 97.79 100.33) (end 99.06 99.06) (width 0.25) (layer F.Cu) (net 23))
 (segment (start 73.66 100.33) (end 97.79 100.33) (width 0.25) (layer F.Cu) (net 23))
 (segment (start 72.39 99.06) (end 73.66 100.33) (width 0.25) (layer F.Cu) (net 23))
 (segment (start 72.39 71.12) (end 72.39 99.06) (width 0.25) (layer F.Cu) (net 23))
 (segment (start 69.85 68.58) (end 72.39 71.12) (width 0.25) (layer F.Cu) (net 23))
 (segment (start 62.23 68.58) (end 66.04 68.58) (width 0.25) (layer F.Cu) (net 23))
 (segment (start 66.04 71.12) (end 69.85 71.12) (width 0.25) (layer B.Cu) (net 24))
 (segment (start 101.6 90.17) (end 105.41 90.17) (width 0.25) (layer B.Cu) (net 24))
 (segment (start 93.98 97.79) (end 101.6 90.17) (width 0.25) (layer B.Cu) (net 24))
 (segment (start 76.2 97.79) (end 93.98 97.79) (width 0.25) (layer B.Cu) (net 24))
 (segment (start 74.93 96.52) (end 76.2 97.79) (width 0.25) (layer B.Cu) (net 24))
 (segment (start 74.93 76.2) (end 74.93 96.52) (width 0.25) (layer B.Cu) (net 24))
 (segment (start 69.85 71.12) (end 74.93 76.2) (width 0.25) (layer B.Cu) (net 24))
 (segment (start 62.23 71.12) (end 66.04 71.12) (width 0.25) (layer F.Cu) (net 24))
 (segment (start 66.04 73.66) (end 69.85 73.66) (width 0.25) (layer B.Cu) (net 25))
 (segment (start 102.87 92.71) (end 105.41 92.71) (width 0.25) (layer B.Cu) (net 25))
 (segment (start 96.52 99.06) (end 102.87 92.71) (width 0.25) (layer B.Cu) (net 25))
 (segment (start 74.93 99.06) (end 96.52 99.06) (width 0.25) (layer B.Cu) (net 25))
 (segment (start 73.66 97.79) (end 74.93 99.06) (width 0.25) (layer B.Cu) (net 25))
 (segment (start 73.66 77.47) (end 73.66 97.79) (width 0.25) (layer B.Cu) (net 25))
 (segment (start 69.85 73.66) (end 73.66 77.47) (width 0.25) (layer B.Cu) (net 25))
 (segment (start 62.23 73.66) (end 66.04 73.66) (width 0.25) (layer F.Cu) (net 25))
 (segment (start 66.04 76.2) (end 69.85 76.2) (width 0.25) (layer B.Cu) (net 26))
 (segment (start 102.87 95.25) (end 105.41 95.25) (width 0.25) (layer B.Cu) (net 26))
 (segment (start 97.79 100.33) (end 102.87 95.25) (width 0.25) (layer B.Cu) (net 26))
 (segment (start 73.66 100.33) (end 97.79 100.33) (width 0.25) (layer B.Cu) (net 26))
 (segment (start 72.39 99.06) (end 73.66 100.33) (width 0.25) (layer B.Cu) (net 26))
 (segment (start 72.39 78.74) (end 72.39 99.06) (width 0.25) (layer B.Cu) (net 26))
 (segment (start 69.85 76.2) (end 72.39 78.74) (width 0.25) (layer B.Cu) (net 26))
 (segment (start 62.23 76.2) (end 66.04 76.2) (width 0.25) (layer F.Cu) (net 26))
 (segment (start 66.04 78.74) (end 68.58 78.74) (width 0.25) (layer B.Cu) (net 27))
 (segment (start 102.87 97.79) (end 105.41 97.79) (width 0.25) (layer B.Cu) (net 27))
 (segment (start 99.06 101.6) (end 102.87 97.79) (width 0.25) (layer B.Cu) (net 27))
 (segment (start 72.39 101.6) (end 99.06 101.6) (width 0.25) (layer B.Cu) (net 27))
 (segment (start 71.12 100.33) (end 72.39 101.6) (width 0.25) (layer B.Cu) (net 27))
 (segment (start 71.12 80.01) (end 71.12 100.33) (width 0.25) (layer B.Cu) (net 27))
 (segment (start 69.85 78.74) (end 71.12 80.01) (width 0.25) (layer B.Cu) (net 27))
 (segment (start 68.58 78.74) (end 69.85 78.74) (width 0.25) (layer B.Cu) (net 27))
 (segment (start 62.23 78.74) (end 66.04 78.74) (width 0.25) (layer F.Cu) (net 27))
 (segment (start 66.04 81.28) (end 69.85 81.28) (width 0.25) (layer B.Cu) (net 28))
 (segment (start 104.14 100.33) (end 105.41 100.33) (width 0.25) (layer B.Cu) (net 28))
 (segment (start 101.6 102.87) (end 104.14 100.33) (width 0.25) (layer B.Cu) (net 28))
 (segment (start 69.85 102.87) (end 101.6 102.87) (width 0.25) (layer B.Cu) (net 28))
 (segment (start 69.85 81.28) (end 69.85 102.87) (width 0.25) (layer B.Cu) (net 28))
 (segment (start 62.23 81.28) (end 66.04 81.28) (width 0.25) (layer F.Cu) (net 28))
 (segment (start 66.04 83.82) (end 68.58 83.82) (width 0.25) (layer B.Cu) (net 29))
 (segment (start 104.14 102.87) (end 105.41 102.87) (width 0.25) (layer B.Cu) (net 29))
 (segment (start 102.87 104.14) (end 104.14 102.87) (width 0.25) (layer B.Cu) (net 29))
 (segment (start 68.58 104.14) (end 102.87 104.14) (width 0.25) (layer B.Cu) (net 29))
 (segment (start 68.58 83.82) (end 68.58 104.14) (width 0.25) (layer B.Cu) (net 29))
 (segment (start 62.23 83.82) (end 66.04 83.82) (width 0.25) (layer F.Cu) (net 29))
 (segment (start 66.04 86.36) (end 67.31 86.36) (width 0.25) (layer B.Cu) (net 30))
 (segment (start 67.31 105.41) (end 105.41 105.41) (width 0.25) (layer B.Cu) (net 30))
 (segment (start 67.31 87.63) (end 67.31 105.41) (width 0.25) (layer B.Cu) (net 30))
 (segment (start 67.31 86.36) (end 67.31 87.63) (width 0.25) (layer B.Cu) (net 30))
 (segment (start 62.23 86.36) (end 66.04 86.36) (width 0.25) (layer F.Cu) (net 30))
 (segment (start 66.04 45.72) (end 69.85 41.91) (width 0.25) (layer F.Cu) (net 12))
 (segment (start 99.06 58.42) (end 100.33 58.42) (width 0.25) (layer F.Cu) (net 12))
 (segment (start 97.79 57.15) (end 99.06 58.42) (width 0.25) (layer F.Cu) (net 12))
 (segment (start 97.79 44.45) (end 97.79 57.15) (width 0.25) (layer F.Cu) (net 12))
 (segment (start 95.25 41.91) (end 97.79 44.45) (width 0.25) (layer F.Cu) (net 12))
 (segment (start 69.85 41.91) (end 95.25 41.91) (width 0.25) (layer F.Cu) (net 12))
 (segment (start 100.33 60.96) (end 100.33 58.42) (width 0.25) (layer F.Cu) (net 12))
 (segment (start 85.09 73.66) (end 87.63 73.66) (width 0.25) (layer F.Cu) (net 12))
 (segment (start 87.63 73.66) (end 91.44 69.85) (width 0.25) (layer F.Cu) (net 12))
 (segment (start 91.44 69.85) (end 91.44 66.04) (width 0.25) (layer F.Cu) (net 12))
 (segment (start 91.44 66.04) (end 96.52 60.96) (width 0.25) (layer F.Cu) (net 12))
 (segment (start 96.52 60.96) (end 100.33 60.96) (width 0.25) (layer F.Cu) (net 12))
 (segment (start 66.04 45.72) (end 66.04 41.91) (width 0.25) (layer B.Cu) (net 12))
 (segment (start 66.04 41.91) (end 62.23 41.91) (width 0.25) (layer B.Cu) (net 12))
 (segment (start 62.23 41.91) (end 62.23 45.72) (width 0.25) (layer B.Cu) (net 12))
 (segment (start 62.23 45.72) (end 66.04 45.72) (width 0.25) (layer F.Cu) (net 12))
 (segment (start 62.23 58.42) (end 66.04 58.42) (width 0.25) (layer F.Cu) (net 31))
 (segment (start 62.23 60.96) (end 66.04 60.96) (width 0.25) (layer F.Cu) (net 32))
 (segment (start 62.23 63.5) (end 66.04 63.5) (width 0.25) (layer F.Cu) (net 33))
 (segment (start 62.23 66.04) (end 66.04 66.04) (width 0.25) (layer F.Cu) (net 34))
 (segment (start 62.23 88.9) (end 66.04 88.9) (width 0.25) (layer F.Cu) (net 35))
 (segment (start 62.23 91.44) (end 66.04 91.44) (width 0.25) (layer F.Cu) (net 36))
 (segment (start 62.23 93.98) (end 60.96 93.98) (width 0.25) (layer F.Cu) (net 22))
 (segment (start 100.33 43.18) (end 100.33 45.72) (width 0.25) (layer F.Cu) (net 22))
 (segment (start 97.79 40.64) (end 100.33 43.18) (width 0.25) (layer F.Cu) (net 22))
 (segment (start 63.5 40.64) (end 97.79 40.64) (width 0.25) (layer F.Cu) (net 22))
 (segment (start 59.69 44.45) (end 63.5 40.64) (width 0.25) (layer F.Cu) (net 22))
 (segment (start 59.69 92.71) (end 59.69 44.45) (width 0.25) (layer F.Cu) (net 22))
 (segment (start 60.96 93.98) (end 59.69 92.71) (width 0.25) (layer F.Cu) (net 22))
 (segment (start 62.23 93.98) (end 62.23 97.79) (width 0.25) (layer B.Cu) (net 22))
 (segment (start 62.23 97.79) (end 66.04 97.79) (width 0.25) (layer B.Cu) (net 22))
 (segment (start 66.04 93.98) (end 66.04 97.79) (width 0.25) (layer B.Cu) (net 22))
 (segment (start 62.23 93.98) (end 66.04 93.98) (width 0.25) (layer F.Cu) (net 22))
 (segment (start 77.47 93.98) (end 81.28 93.98) (width 0.25) (layer F.Cu) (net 37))
 (segment (start 77.47 91.44) (end 81.28 91.44) (width 0.25) (layer F.Cu) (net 38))
 (segment (start 77.47 88.9) (end 81.28 88.9) (width 0.25) (layer F.Cu) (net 39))
 (segment (start 77.47 86.36) (end 81.28 86.36) (width 0.25) (layer F.Cu) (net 40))
 (segment (start 77.47 83.82) (end 81.28 83.82) (width 0.25) (layer F.Cu) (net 41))
 (segment (start 77.47 81.28) (end 81.28 81.28) (width 0.25) (layer F.Cu) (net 42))
 (segment (start 77.47 78.74) (end 81.28 78.74) (width 0.25) (layer F.Cu) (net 43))
 (segment (start 77.47 76.2) (end 81.28 76.2) (width 0.25) (layer F.Cu) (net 44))
 (segment (start 77.47 73.66) (end 81.28 73.66) (width 0.25) (layer F.Cu) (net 45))
 (segment (start 77.47 71.12) (end 81.28 71.12) (width 0.25) (layer F.Cu) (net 46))
 (segment (start 77.47 68.58) (end 81.28 68.58) (width 0.25) (layer F.Cu) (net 47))
 (segment (start 77.47 66.04) (end 81.28 66.04) (width 0.25) (layer F.Cu) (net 48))
 (segment (start 77.47 63.5) (end 81.28 63.5) (width 0.25) (layer F.Cu) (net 49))
 (segment (start 77.47 60.96) (end 81.28 60.96) (width 0.25) (layer F.Cu) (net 50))
 (segment (start 77.47 58.42) (end 81.28 58.42) (width 0.25) (layer F.Cu) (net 51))
 (segment (start 77.47 55.88) (end 81.28 55.88) (width 0.25) (layer F.Cu) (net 52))
 (segment (start 77.47 53.34) (end 81.28 53.34) (width 0.25) (layer F.Cu) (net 53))
 (segment (start 77.47 50.8) (end 81.28 50.8) (width 0.25) (layer F.Cu) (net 54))
 (segment (start 77.47 48.26) (end 81.28 48.26) (width 0.25) (layer F.Cu) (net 55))
 (segment (start 77.47 45.72) (end 81.28 45.72) (width 0.25) (layer F.Cu) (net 56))
 (segment (start 66.04 48.26) (end 67.31 48.26) (width 0.25) (layer B.Cu) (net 21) (status 400000))
 (segment (start 87.63 48.26) (end 100.33 48.26) (width 0.25) (layer B.Cu) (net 21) (status 800000))
 (segment (start 86.36 49.53) (end 87.63 48.26) (width 0.25) (layer B.Cu) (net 21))
 (segment (start 68.58 49.53) (end 86.36 49.53) (width 0.25) (layer B.Cu) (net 21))
 (segment (start 67.31 48.26) (end 68.58 49.53) (width 0.25) (layer B.Cu) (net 21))
 (segment (start 62.23 48.26) (end 66.04 48.26) (width 0.25) (layer F.Cu) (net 21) (status C00000))
 (segment (start 66.04 50.8) (end 67.31 50.8) (width 0.25) (layer B.Cu) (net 20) (status 400000))
 (segment (start 87.63 50.8) (end 100.33 50.8) (width 0.25) (layer B.Cu) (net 20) (status 800000))
 (segment (start 86.36 52.07) (end 87.63 50.8) (width 0.25) (layer B.Cu) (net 20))
 (segment (start 68.58 52.07) (end 86.36 52.07) (width 0.25) (layer B.Cu) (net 20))
 (segment (start 67.31 50.8) (end 68.58 52.07) (width 0.25) (layer B.Cu) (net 20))
 (segment (start 62.23 50.8) (end 66.04 50.8) (width 0.25) (layer F.Cu) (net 20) (status C00000))
 (segment (start 66.04 53.34) (end 67.31 53.34) (width 0.25) (layer B.Cu) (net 19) (status 400000))
 (segment (start 87.63 53.34) (end 100.33 53.34) (width 0.25) (layer B.Cu) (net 19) (status 800000))
 (segment (start 86.36 54.61) (end 87.63 53.34) (width 0.25) (layer B.Cu) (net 19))
 (segment (start 68.58 54.61) (end 86.36 54.61) (width 0.25) (layer B.Cu) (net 19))
 (segment (start 67.31 53.34) (end 68.58 54.61) (width 0.25) (layer B.Cu) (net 19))
 (segment (start 62.23 53.34) (end 66.04 53.34) (width 0.25) (layer F.Cu) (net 19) (status C00000))
 (segment (start 66.04 55.88) (end 67.31 55.88) (width 0.25) (layer B.Cu) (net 18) (status 400000))
 (segment (start 87.63 55.88) (end 100.33 55.88) (width 0.25) (layer B.Cu) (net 18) (status 800000))
 (segment (start 86.36 57.15) (end 87.63 55.88) (width 0.25) (layer B.Cu) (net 18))
 (segment (start 68.58 57.15) (end 86.36 57.15) (width 0.25) (layer B.Cu) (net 18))
 (segment (start 67.31 55.88) (end 68.58 57.15) (width 0.25) (layer B.Cu) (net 18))
 (segment (start 62.23 55.88) (end 66.04 55.88) (width 0.25) (layer F.Cu) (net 18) (status C00000)))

